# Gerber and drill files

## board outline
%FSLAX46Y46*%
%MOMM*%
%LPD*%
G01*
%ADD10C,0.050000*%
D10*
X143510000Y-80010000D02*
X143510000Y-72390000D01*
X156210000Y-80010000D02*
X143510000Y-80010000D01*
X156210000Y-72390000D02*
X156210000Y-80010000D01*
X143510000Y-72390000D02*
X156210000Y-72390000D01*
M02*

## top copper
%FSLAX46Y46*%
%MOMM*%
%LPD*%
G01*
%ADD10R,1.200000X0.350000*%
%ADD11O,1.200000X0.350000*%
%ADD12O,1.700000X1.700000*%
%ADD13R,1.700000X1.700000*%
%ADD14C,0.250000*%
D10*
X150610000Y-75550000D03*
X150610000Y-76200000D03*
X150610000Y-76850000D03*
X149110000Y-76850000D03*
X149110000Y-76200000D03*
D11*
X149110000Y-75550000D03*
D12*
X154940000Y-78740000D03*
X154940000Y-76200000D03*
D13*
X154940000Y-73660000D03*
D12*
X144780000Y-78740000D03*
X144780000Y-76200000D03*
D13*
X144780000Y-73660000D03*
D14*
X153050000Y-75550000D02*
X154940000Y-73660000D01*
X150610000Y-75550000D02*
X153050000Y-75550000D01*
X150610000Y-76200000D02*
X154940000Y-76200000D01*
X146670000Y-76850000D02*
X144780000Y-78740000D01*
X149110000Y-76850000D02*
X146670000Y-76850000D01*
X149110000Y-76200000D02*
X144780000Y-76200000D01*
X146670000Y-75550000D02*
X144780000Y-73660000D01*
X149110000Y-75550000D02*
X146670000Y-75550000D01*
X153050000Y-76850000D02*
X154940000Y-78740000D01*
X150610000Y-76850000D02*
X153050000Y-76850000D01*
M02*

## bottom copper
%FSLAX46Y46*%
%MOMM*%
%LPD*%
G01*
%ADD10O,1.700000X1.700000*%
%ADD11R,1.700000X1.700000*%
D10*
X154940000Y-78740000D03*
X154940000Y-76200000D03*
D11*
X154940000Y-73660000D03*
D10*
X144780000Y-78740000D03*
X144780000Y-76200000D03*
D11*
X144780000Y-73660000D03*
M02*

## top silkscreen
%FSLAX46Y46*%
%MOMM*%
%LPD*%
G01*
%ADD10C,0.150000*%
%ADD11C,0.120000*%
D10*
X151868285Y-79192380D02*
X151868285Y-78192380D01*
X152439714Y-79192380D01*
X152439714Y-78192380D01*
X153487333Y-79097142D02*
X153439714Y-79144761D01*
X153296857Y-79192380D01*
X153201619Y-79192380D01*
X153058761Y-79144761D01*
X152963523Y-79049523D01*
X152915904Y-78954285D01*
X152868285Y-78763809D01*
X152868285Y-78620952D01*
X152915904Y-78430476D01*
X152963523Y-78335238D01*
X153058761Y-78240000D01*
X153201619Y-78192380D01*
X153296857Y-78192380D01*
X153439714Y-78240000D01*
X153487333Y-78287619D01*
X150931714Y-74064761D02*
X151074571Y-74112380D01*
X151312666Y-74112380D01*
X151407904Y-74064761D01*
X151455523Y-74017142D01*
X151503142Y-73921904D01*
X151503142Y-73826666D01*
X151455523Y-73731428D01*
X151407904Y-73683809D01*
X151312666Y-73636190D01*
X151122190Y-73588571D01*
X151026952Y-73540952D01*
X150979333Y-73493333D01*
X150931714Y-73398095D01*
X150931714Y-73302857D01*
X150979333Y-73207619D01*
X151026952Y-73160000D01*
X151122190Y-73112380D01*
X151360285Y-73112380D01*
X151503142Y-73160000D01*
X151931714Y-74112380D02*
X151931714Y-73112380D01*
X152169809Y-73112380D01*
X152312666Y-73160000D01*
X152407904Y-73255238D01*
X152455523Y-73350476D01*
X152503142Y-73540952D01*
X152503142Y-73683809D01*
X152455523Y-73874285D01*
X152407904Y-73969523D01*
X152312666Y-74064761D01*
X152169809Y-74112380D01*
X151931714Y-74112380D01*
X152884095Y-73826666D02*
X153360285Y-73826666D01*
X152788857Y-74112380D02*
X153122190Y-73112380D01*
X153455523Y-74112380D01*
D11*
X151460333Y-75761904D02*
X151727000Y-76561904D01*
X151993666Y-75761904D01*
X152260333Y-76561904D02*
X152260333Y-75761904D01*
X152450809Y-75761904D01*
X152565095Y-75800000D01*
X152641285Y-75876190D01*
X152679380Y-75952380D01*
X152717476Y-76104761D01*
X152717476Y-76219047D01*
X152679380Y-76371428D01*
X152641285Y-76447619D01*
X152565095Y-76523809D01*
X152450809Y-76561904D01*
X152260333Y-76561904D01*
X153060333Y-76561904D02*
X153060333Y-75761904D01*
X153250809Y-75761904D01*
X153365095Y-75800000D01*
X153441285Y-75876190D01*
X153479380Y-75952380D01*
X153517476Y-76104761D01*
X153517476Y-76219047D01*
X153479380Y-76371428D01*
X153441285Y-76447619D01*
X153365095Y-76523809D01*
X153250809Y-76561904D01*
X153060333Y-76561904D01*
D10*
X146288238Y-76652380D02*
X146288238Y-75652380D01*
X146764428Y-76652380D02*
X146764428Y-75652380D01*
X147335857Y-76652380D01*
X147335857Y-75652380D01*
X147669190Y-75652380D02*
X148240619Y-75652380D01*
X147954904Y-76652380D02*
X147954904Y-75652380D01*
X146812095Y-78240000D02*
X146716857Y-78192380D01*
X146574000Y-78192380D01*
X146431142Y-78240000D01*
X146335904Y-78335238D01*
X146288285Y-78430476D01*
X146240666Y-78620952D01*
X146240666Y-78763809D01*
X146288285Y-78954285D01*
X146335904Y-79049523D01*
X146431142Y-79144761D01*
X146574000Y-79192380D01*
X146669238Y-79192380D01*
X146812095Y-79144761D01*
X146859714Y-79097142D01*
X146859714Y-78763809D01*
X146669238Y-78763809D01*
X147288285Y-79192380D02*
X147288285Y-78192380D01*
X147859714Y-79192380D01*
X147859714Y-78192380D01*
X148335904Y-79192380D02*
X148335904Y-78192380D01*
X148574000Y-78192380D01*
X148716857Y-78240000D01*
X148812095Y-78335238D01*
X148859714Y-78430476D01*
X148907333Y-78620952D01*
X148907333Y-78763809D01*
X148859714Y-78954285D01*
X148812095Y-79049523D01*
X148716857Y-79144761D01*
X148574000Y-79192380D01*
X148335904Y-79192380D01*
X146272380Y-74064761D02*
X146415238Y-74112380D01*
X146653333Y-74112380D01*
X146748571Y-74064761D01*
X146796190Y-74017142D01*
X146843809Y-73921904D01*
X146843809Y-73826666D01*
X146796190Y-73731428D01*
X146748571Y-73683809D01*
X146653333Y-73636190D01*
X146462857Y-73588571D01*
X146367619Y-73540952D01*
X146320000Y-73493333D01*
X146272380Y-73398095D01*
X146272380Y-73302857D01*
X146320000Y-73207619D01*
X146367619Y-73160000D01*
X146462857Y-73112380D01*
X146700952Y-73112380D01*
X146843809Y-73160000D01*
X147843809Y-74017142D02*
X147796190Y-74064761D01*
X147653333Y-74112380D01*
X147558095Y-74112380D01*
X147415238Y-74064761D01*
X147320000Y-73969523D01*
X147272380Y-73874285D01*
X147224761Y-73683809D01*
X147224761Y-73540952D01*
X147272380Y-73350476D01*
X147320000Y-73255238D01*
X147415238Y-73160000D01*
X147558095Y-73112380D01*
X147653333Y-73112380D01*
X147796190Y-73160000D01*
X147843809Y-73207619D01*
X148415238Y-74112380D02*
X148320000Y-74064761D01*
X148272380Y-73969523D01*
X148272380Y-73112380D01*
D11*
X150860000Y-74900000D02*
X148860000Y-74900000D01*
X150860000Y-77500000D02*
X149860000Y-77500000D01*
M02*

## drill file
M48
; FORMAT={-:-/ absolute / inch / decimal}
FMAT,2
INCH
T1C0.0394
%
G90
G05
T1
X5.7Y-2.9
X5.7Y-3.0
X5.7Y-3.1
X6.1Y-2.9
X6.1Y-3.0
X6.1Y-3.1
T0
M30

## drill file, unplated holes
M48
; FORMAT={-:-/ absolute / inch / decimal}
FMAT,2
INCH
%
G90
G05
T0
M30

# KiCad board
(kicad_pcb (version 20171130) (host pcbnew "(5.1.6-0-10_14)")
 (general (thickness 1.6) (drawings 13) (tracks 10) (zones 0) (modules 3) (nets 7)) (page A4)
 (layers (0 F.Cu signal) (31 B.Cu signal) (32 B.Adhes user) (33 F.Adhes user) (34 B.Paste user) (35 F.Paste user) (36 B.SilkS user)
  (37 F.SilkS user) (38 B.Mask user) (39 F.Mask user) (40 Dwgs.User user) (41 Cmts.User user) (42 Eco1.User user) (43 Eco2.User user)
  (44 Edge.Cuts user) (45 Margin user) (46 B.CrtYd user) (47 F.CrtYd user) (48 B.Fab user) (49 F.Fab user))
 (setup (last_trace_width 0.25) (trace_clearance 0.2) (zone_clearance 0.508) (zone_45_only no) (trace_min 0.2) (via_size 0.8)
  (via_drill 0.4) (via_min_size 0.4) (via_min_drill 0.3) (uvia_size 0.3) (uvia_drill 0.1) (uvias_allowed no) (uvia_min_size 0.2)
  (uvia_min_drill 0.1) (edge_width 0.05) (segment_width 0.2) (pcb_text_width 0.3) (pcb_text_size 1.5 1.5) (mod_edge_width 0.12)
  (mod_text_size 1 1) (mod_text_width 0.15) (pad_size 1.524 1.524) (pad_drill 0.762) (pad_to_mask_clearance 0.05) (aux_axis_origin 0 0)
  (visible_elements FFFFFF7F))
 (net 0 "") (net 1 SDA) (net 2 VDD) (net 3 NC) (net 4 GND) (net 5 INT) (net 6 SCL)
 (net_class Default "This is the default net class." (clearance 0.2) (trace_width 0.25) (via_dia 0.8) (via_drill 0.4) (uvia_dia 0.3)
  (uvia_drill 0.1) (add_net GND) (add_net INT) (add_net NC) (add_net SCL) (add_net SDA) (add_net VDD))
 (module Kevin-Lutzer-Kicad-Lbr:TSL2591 (layer F.Cu) (at 149.86 76.2)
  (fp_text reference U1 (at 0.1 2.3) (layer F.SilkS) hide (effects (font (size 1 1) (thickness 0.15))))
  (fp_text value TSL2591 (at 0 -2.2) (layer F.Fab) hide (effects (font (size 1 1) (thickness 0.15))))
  (fp_line (start 1 1.3) (end 0 1.3) (layer F.SilkS) (width 0.12))
  (fp_line (start 1 -1.3) (end -1 -1.3) (layer F.SilkS) (width 0.12))
  (pad 6 smd rect (at 0.75 -0.65) (size 1.2 0.35) (layers F.Cu F.Paste F.Mask) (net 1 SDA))
  (pad 5 smd rect (at 0.75 0) (size 1.2 0.35) (layers F.Cu F.Paste F.Mask) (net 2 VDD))
  (pad 4 smd rect (at 0.75 0.65) (size 1.2 0.35) (layers F.Cu F.Paste F.Mask) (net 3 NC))
  (pad 3 smd rect (at -0.75 0.65) (size 1.2 0.35) (layers F.Cu F.Paste F.Mask) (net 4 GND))
  (pad 2 smd rect (at -0.75 0) (size 1.2 0.35) (layers F.Cu F.Paste F.Mask) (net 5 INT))
  (pad 1 smd oval (at -0.75 -0.65) (size 1.2 0.35) (layers F.Cu F.Paste F.Mask) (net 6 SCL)))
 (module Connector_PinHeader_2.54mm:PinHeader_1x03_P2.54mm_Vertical (layer B.Cu) (at 154.94 73.66 180)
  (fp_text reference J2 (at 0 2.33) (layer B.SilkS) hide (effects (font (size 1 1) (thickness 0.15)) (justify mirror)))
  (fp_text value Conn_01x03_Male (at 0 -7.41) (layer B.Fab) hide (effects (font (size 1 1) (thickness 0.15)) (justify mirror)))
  (pad 3 thru_hole oval (at 0 -5.08 180) (size 1.7 1.7) (drill 1) (layers *.Cu *.Mask) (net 3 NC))
  (pad 2 thru_hole oval (at 0 -2.54 180) (size 1.7 1.7) (drill 1) (layers *.Cu *.Mask) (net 2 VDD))
  (pad 1 thru_hole rect (at 0 0 180) (size 1.7 1.7) (drill 1) (layers *.Cu *.Mask) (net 1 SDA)))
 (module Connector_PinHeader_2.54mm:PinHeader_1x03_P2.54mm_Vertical (layer B.Cu) (at 144.78 73.66 180)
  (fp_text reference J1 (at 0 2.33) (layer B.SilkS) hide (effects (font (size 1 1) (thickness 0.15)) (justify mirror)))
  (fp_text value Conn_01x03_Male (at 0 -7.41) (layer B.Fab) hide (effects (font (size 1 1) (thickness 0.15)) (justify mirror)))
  (pad 3 thru_hole oval (at 0 -5.08 180) (size 1.7 1.7) (drill 1) (layers *.Cu *.Mask) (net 4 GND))
  (pad 2 thru_hole oval (at 0 -2.54 180) (size 1.7 1.7) (drill 1) (layers *.Cu *.Mask) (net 5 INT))
  (pad 1 thru_hole rect (at 0 0 180) (size 1.7 1.7) (drill 1) (layers *.Cu *.Mask) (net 6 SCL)))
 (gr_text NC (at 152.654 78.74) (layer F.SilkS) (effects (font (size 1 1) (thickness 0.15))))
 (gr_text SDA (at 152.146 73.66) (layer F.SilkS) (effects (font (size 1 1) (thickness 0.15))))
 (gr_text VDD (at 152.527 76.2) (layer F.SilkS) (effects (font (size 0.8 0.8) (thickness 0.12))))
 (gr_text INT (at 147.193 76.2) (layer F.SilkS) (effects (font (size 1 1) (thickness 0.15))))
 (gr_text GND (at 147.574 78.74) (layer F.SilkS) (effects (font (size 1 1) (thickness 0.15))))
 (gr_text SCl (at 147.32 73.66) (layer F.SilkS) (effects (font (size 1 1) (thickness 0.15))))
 (gr_line (start 143.51 80.01) (end 143.51 72.39) (layer Edge.Cuts) (width 0.05))
 (gr_line (start 156.21 80.01) (end 143.51 80.01) (layer Edge.Cuts) (width 0.05))
 (gr_line (start 156.21 72.39) (end 156.21 80.01) (layer Edge.Cuts) (width 0.05))
 (gr_line (start 143.51 72.39) (end 156.21 72.39) (layer Edge.Cuts) (width 0.05))
 (segment (start 153.05 75.55) (end 154.94 73.66) (width 0.25) (layer F.Cu) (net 1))
 (segment (start 150.61 75.55) (end 153.05 75.55) (width 0.25) (layer F.Cu) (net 1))
 (segment (start 150.61 76.2) (end 154.94 76.2) (width 0.25) (layer F.Cu) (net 2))
 (segment (start 146.67 76.85) (end 144.78 78.74) (width 0.25) (layer F.Cu) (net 4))
 (segment (start 149.11 76.85) (end 146.67 76.85) (width 0.25) (layer F.Cu) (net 4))
 (segment (start 149.11 76.2) (end 144.78 76.2) (width 0.25) (layer F.Cu) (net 5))
 (segment (start 146.67 75.55) (end 144.78 73.66) (width 0.25) (layer F.Cu) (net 6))
 (segment (start 149.11 75.55) (end 146.67 75.55) (width 0.25) (layer F.Cu) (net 6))
 (segment (start 153.05 76.85) (end 154.94 78.74) (width 0.25) (layer F.Cu) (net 3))
 (segment (start 150.61 76.85) (end 153.05 76.85) (width 0.25) (layer F.Cu) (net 3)))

